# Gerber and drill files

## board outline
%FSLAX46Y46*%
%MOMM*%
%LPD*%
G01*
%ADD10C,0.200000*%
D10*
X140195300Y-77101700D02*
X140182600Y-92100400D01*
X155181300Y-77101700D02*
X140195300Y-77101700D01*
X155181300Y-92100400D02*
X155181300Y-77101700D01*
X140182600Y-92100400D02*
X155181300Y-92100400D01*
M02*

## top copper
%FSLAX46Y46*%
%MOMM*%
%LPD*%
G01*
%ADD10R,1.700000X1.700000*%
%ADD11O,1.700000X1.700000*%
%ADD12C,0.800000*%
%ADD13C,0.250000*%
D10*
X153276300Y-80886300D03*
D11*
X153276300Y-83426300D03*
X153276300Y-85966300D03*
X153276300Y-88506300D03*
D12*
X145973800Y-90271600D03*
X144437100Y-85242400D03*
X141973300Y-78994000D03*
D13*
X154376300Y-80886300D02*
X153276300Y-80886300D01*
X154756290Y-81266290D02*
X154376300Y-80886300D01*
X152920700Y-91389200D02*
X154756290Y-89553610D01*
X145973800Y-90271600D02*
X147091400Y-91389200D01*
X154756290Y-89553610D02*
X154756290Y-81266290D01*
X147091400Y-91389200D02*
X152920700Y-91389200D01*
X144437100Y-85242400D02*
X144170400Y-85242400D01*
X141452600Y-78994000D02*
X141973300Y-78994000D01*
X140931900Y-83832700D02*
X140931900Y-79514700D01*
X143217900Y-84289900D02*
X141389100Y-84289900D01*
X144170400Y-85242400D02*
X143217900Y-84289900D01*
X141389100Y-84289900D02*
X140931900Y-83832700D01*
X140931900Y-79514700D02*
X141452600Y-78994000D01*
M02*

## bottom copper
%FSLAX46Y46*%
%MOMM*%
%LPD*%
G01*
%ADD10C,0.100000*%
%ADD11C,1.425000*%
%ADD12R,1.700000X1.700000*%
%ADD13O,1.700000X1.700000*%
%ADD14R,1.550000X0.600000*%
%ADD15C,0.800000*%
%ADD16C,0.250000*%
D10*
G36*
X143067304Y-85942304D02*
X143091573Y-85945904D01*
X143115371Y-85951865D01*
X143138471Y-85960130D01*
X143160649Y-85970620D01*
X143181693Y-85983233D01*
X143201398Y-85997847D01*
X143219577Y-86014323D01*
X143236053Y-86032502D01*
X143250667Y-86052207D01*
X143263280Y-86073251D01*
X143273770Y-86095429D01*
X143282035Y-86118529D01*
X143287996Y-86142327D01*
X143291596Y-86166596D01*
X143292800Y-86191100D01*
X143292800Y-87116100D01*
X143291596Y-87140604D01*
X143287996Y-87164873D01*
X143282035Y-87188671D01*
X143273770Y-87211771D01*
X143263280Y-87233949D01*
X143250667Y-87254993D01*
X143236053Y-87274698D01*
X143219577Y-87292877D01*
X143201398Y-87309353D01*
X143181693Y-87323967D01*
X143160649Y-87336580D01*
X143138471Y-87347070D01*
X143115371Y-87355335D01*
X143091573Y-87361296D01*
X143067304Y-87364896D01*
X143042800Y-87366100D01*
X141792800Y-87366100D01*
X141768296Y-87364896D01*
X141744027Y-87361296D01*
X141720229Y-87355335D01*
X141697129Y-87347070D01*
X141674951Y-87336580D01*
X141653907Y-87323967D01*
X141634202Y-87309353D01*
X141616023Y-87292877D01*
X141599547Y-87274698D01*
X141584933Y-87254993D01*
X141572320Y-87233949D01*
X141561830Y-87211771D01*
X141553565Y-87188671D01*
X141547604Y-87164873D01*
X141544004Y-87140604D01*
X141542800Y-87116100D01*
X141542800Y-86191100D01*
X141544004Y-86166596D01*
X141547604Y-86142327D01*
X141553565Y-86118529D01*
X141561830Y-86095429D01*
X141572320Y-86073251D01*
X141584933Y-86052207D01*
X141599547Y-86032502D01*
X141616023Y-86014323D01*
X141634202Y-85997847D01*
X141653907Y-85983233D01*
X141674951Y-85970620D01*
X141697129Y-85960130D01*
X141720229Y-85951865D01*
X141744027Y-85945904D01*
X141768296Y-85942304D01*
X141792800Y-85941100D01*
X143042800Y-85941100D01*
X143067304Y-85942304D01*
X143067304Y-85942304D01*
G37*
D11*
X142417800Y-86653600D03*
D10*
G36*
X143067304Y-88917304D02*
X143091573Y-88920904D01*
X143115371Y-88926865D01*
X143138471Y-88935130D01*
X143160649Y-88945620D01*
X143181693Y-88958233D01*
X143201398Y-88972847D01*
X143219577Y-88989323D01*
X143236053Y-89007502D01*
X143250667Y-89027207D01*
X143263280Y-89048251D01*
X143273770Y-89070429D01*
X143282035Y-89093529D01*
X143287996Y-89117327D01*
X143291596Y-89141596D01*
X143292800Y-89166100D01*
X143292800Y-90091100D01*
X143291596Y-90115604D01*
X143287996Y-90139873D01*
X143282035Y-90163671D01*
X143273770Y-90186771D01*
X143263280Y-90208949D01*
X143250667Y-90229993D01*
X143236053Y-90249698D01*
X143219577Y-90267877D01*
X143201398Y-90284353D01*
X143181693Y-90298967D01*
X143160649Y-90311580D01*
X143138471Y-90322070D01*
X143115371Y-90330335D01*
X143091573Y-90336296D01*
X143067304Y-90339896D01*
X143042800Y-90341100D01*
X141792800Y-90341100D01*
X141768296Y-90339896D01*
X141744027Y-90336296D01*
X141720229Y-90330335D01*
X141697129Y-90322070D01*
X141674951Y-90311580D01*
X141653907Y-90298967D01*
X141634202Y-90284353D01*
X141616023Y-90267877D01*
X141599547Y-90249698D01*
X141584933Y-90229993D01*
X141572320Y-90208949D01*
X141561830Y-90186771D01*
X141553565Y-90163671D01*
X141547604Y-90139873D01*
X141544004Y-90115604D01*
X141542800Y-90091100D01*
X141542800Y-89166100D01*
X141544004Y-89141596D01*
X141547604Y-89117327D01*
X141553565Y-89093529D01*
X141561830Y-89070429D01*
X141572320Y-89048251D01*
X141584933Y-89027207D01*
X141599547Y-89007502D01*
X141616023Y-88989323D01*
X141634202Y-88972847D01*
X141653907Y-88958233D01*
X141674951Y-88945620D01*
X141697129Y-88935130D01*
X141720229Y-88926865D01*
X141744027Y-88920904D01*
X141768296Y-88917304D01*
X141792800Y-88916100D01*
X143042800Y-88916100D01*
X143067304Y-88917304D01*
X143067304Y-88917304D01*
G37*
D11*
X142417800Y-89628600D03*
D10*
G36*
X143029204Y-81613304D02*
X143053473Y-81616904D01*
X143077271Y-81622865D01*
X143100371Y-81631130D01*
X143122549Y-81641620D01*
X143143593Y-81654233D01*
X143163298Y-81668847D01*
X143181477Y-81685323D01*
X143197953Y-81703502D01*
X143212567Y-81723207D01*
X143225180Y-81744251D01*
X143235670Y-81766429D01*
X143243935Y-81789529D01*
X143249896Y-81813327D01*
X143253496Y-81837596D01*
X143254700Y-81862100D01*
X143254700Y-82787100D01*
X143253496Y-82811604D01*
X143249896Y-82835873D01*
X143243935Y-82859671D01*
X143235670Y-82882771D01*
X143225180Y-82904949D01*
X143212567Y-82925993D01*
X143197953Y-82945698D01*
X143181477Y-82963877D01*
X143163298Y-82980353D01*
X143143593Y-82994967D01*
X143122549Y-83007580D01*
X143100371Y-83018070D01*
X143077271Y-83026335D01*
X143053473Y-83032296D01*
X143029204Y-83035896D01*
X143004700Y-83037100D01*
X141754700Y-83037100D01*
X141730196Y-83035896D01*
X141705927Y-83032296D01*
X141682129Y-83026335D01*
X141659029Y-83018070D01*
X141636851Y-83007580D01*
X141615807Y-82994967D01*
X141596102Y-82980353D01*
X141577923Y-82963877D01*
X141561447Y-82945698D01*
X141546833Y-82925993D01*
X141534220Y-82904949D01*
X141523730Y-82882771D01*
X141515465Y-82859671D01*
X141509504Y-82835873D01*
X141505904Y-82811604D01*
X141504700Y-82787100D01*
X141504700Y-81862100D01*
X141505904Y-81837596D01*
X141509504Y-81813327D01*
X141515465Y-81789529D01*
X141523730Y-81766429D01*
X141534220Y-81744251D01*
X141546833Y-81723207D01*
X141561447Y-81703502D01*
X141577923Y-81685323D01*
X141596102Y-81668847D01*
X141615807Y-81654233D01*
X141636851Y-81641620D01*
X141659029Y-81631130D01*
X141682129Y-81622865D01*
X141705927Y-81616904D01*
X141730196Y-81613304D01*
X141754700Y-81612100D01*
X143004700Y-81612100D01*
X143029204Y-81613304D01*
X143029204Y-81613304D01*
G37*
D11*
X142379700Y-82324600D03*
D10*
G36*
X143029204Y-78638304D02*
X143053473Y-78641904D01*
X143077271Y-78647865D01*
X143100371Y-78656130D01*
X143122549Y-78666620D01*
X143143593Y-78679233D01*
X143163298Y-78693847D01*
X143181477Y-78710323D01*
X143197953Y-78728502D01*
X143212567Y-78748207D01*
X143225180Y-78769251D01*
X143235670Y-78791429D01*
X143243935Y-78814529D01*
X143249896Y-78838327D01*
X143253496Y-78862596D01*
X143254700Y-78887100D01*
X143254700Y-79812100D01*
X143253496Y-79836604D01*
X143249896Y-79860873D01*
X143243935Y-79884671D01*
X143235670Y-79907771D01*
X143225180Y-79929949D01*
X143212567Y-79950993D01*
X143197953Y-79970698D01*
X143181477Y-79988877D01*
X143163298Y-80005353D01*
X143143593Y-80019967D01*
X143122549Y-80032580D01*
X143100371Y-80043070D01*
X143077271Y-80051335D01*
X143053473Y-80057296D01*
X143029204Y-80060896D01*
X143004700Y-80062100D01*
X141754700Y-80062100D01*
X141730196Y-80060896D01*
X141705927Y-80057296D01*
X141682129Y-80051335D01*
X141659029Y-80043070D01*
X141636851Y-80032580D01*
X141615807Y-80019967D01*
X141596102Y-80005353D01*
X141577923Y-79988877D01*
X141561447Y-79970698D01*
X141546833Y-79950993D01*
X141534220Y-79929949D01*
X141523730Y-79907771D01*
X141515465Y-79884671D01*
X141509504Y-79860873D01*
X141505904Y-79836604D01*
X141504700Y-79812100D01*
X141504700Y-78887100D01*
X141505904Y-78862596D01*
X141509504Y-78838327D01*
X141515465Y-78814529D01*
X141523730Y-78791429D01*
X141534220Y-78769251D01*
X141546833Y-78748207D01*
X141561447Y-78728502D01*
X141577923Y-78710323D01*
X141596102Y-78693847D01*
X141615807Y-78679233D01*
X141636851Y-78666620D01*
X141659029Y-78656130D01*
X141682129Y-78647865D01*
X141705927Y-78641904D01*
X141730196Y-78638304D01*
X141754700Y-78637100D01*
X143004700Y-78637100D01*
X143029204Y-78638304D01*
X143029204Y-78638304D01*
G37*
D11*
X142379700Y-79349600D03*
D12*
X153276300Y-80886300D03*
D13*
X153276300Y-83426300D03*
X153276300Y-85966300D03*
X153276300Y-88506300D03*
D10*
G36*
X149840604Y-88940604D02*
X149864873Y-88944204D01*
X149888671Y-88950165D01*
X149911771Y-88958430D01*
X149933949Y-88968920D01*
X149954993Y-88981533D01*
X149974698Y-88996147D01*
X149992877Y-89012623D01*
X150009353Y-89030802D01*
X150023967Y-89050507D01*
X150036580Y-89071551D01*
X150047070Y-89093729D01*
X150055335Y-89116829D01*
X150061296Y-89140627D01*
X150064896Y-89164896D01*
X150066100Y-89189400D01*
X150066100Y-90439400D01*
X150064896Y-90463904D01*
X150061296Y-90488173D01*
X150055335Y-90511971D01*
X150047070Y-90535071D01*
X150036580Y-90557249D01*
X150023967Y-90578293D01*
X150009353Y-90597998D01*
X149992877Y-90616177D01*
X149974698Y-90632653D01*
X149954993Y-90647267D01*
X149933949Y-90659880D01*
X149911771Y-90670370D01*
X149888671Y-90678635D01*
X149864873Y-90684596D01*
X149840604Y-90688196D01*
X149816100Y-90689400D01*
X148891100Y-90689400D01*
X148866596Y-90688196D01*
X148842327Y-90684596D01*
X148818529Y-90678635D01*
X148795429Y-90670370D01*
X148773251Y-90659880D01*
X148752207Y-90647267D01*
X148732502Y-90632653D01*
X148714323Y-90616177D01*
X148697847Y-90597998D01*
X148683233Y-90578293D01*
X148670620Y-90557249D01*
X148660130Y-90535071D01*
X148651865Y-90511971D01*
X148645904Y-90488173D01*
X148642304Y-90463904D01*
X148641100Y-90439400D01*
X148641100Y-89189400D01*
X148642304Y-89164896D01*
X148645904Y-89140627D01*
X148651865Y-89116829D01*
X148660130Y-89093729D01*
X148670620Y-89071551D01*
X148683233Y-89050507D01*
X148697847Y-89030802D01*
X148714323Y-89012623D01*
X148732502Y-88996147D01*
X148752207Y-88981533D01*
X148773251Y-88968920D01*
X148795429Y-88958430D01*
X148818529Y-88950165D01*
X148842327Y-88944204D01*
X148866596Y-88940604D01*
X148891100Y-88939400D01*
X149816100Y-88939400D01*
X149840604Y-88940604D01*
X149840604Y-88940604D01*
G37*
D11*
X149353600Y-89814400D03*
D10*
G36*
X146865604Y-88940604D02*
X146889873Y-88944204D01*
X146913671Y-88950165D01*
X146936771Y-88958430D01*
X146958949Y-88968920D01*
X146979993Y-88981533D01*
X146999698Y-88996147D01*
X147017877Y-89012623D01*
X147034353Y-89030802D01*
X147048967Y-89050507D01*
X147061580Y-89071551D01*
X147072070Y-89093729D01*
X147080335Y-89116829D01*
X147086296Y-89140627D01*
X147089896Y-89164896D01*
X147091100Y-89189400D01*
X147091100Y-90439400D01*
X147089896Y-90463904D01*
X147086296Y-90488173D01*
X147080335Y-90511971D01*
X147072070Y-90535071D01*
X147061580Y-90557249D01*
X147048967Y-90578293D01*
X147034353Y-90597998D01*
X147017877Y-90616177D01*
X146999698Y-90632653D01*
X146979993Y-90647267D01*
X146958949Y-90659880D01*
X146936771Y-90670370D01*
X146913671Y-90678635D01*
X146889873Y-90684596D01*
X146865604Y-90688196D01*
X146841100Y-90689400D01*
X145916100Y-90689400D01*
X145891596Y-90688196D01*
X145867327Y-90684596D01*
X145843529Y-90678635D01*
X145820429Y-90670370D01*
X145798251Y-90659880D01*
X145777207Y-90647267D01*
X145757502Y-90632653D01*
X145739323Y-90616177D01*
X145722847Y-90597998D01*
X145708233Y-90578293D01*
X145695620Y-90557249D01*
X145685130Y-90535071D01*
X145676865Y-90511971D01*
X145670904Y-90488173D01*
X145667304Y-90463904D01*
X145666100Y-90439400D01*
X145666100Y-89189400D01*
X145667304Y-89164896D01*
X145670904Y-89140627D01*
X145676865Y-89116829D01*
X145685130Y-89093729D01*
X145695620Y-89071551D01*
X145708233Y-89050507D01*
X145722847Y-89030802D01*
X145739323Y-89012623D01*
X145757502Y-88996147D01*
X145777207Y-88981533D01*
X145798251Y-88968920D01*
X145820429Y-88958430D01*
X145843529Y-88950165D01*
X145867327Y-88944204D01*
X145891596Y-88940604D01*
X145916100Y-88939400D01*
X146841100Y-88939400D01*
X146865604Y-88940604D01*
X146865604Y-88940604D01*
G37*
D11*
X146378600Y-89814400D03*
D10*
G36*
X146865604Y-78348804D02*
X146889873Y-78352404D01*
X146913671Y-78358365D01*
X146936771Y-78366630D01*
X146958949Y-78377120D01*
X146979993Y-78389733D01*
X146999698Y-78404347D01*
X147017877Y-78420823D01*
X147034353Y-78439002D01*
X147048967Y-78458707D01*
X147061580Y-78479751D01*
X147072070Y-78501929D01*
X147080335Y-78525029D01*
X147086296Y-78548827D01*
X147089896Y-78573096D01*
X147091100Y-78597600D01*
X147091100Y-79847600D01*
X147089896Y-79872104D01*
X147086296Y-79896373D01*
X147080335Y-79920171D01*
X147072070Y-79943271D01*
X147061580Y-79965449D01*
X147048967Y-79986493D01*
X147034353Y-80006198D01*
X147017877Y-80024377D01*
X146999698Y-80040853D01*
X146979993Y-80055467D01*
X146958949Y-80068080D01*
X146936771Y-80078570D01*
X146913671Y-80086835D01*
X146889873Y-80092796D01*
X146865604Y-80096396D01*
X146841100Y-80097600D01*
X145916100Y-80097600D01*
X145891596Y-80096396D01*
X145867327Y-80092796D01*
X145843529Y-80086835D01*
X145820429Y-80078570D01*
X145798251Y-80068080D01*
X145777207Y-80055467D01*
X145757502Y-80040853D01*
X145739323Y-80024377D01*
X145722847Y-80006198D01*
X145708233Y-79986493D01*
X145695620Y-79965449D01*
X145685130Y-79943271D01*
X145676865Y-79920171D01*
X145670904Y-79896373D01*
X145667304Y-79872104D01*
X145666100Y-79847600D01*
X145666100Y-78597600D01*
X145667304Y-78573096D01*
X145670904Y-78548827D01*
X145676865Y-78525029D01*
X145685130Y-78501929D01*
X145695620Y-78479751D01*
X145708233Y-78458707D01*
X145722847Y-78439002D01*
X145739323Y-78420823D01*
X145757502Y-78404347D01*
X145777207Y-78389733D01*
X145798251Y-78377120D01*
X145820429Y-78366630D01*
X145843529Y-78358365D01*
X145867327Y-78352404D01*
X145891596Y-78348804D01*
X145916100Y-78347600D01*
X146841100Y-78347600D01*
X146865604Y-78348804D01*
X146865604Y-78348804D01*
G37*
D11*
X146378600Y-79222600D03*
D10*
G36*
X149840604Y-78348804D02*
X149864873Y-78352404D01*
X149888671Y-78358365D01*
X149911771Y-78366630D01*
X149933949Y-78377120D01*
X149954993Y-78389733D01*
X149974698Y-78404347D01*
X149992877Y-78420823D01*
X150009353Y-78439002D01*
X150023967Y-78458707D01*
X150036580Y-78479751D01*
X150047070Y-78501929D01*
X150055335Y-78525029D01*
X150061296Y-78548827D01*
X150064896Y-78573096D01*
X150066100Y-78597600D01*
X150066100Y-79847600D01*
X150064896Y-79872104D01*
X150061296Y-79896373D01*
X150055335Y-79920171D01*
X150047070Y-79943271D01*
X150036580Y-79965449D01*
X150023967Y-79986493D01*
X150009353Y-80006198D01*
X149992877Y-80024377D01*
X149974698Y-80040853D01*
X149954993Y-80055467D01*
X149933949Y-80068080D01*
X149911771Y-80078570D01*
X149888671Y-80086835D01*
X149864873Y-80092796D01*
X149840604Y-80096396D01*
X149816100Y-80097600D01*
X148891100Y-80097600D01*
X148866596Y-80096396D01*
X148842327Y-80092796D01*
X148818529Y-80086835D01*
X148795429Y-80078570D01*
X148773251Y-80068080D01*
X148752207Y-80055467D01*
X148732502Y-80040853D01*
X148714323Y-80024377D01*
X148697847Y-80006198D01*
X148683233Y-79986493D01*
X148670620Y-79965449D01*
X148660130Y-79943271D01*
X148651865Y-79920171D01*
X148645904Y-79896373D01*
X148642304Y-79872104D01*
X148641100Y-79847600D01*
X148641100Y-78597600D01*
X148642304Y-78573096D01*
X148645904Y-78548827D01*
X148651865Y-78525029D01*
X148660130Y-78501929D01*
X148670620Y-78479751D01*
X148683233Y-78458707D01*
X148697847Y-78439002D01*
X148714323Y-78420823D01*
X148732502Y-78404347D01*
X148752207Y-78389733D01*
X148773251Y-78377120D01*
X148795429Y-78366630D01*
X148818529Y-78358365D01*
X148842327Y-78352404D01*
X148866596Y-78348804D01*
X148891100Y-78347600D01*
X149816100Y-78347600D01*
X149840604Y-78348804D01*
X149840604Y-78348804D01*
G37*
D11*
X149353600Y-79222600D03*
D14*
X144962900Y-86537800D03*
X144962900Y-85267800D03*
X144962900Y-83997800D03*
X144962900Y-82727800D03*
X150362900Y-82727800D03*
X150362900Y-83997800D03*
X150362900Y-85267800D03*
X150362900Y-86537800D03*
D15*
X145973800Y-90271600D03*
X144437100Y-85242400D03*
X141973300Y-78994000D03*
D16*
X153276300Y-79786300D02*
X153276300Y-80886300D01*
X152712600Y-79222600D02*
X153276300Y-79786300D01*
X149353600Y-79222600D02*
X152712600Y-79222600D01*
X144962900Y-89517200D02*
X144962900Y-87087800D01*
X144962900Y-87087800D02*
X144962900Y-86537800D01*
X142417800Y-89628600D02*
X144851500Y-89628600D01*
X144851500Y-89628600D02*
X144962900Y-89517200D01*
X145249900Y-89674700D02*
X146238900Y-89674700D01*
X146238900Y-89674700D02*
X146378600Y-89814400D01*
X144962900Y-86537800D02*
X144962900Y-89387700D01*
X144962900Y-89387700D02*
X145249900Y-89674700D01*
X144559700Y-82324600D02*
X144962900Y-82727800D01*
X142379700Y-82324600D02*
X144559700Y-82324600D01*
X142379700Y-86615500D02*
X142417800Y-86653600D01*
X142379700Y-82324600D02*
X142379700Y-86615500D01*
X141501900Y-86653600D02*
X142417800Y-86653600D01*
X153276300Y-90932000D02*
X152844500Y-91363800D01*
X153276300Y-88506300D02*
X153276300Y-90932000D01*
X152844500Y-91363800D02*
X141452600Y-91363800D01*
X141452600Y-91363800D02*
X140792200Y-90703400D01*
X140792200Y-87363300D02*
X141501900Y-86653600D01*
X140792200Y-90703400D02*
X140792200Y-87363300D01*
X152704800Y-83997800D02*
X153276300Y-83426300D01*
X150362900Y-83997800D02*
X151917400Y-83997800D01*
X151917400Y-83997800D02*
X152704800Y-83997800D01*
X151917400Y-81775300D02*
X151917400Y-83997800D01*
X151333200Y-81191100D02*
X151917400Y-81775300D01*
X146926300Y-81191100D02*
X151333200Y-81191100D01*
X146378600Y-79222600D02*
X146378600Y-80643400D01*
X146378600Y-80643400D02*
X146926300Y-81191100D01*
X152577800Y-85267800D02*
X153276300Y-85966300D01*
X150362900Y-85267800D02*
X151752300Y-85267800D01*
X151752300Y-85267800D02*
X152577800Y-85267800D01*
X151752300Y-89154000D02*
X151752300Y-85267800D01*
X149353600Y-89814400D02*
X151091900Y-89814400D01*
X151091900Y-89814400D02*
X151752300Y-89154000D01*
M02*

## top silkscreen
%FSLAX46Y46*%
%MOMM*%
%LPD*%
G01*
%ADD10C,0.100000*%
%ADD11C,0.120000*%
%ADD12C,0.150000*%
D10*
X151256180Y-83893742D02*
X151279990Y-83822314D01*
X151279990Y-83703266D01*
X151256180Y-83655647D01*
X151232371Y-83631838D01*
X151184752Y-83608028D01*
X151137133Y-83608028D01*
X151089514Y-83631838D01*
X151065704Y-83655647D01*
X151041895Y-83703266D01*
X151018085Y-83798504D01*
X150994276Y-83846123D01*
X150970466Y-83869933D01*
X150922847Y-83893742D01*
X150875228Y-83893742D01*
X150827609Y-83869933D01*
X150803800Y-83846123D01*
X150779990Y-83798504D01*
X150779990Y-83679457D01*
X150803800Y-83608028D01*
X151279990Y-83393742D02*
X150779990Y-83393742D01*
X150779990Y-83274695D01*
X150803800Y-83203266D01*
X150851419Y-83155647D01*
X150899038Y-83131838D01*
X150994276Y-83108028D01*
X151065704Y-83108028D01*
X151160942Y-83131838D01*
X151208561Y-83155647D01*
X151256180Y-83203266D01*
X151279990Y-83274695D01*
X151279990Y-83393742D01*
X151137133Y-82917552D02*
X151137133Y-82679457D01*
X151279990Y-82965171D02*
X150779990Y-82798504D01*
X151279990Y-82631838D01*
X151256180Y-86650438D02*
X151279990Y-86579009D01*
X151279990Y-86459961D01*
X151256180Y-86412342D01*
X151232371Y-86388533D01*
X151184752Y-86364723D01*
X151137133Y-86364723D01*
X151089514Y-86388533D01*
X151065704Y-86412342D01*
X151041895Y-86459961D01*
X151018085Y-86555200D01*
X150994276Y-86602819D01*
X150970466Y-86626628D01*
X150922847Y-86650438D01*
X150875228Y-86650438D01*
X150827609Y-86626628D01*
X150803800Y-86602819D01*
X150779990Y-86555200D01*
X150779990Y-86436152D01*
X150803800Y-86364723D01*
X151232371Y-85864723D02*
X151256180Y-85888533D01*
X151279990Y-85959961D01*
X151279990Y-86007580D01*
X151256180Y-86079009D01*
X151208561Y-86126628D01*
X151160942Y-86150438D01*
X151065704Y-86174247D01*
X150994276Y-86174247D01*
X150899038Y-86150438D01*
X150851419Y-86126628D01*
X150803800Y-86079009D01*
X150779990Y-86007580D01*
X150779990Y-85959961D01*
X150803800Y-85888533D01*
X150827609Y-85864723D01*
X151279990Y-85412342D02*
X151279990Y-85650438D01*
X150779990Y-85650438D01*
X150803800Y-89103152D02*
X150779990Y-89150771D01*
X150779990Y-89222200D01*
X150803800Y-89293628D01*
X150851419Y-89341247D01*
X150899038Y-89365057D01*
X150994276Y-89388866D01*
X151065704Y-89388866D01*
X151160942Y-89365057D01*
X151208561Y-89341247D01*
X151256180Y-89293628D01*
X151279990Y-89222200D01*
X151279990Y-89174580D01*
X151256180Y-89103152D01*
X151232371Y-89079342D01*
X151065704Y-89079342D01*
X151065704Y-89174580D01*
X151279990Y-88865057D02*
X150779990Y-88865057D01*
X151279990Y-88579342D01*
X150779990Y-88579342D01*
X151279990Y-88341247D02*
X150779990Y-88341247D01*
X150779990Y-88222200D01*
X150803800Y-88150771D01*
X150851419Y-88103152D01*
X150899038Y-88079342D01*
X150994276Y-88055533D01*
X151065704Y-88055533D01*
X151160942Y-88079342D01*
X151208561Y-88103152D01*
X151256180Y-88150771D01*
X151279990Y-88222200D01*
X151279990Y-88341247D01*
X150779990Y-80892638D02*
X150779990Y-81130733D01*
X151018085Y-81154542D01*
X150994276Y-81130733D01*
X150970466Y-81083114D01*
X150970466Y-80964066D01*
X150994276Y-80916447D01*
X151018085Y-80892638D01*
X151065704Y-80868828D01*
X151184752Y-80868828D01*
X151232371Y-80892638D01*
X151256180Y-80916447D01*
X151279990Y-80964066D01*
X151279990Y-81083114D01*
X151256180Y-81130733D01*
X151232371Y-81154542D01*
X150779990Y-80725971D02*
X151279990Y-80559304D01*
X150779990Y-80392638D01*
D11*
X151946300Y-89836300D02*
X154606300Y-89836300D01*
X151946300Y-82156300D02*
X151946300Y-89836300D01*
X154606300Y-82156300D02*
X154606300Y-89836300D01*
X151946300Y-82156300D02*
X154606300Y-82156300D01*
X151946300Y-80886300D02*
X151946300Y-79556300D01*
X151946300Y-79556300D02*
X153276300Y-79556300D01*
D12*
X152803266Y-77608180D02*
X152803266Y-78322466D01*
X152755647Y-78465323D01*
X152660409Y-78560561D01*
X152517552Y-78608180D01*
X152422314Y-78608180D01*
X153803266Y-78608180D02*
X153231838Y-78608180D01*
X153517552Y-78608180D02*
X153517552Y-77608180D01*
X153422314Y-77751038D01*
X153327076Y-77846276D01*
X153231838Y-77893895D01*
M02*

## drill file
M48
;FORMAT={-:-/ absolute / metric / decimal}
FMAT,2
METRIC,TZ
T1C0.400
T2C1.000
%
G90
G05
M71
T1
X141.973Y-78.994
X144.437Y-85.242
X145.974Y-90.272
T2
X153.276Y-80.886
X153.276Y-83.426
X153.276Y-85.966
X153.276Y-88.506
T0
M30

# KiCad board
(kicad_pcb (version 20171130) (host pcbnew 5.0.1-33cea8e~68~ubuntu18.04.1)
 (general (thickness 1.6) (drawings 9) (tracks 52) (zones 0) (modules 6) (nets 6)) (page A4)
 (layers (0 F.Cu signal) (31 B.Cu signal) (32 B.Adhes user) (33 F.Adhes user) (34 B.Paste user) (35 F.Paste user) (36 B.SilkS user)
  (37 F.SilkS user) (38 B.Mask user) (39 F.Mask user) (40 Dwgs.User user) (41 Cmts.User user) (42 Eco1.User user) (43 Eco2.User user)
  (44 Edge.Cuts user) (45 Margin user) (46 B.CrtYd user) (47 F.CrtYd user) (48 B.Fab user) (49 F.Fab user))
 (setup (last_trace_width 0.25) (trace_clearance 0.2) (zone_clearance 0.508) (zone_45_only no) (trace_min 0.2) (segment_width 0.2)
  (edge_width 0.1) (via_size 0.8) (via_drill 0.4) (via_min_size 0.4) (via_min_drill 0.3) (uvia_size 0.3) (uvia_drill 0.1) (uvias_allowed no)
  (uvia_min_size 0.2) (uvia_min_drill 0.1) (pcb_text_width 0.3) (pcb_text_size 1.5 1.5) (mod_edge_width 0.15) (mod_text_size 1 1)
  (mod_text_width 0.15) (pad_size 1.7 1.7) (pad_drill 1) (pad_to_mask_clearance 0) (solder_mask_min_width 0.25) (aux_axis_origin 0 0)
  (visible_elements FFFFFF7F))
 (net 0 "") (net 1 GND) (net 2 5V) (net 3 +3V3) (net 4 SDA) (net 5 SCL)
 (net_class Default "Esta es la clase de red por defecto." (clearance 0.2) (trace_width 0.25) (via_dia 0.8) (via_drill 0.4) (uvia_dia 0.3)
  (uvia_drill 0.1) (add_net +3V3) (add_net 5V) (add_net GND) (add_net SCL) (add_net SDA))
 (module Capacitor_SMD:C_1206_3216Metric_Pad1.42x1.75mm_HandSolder (layer B.Cu) (at 142.4178 88.1411 90)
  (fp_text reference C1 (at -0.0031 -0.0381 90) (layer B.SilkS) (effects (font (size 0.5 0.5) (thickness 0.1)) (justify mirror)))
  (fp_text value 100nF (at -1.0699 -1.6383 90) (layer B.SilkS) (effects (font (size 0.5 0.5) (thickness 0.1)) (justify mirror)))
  (pad 2 smd roundrect (at 1.4875 0 90) (size 1.425 1.75) (layers B.Cu B.Paste B.Mask) (roundrect_rratio 0.175439) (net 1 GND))
  (pad 1 smd roundrect (at -1.4875 0 90) (size 1.425 1.75) (layers B.Cu B.Paste B.Mask) (roundrect_rratio 0.175439) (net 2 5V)))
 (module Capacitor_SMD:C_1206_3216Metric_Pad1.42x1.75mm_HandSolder (layer B.Cu) (at 142.3797 80.8371 270)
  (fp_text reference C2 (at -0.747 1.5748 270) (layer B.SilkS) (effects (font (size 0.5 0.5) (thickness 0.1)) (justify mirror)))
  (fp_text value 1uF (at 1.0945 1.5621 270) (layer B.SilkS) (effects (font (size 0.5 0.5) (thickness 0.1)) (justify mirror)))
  (pad 2 smd roundrect (at 1.4875 0 270) (size 1.425 1.75) (layers B.Cu B.Paste B.Mask) (roundrect_rratio 0.175439) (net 1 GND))
  (pad 1 smd roundrect (at -1.4875 0 270) (size 1.425 1.75) (layers B.Cu B.Paste B.Mask) (roundrect_rratio 0.175439) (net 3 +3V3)))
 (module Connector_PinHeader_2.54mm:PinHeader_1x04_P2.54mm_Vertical (layer F.Cu) (at 153.2763 80.8863)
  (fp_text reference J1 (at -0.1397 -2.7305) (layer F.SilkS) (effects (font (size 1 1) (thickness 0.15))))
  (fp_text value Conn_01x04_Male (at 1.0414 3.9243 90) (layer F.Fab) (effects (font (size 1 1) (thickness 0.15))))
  (fp_line (start -1.33 8.95) (end 1.33 8.95) (layer F.SilkS) (width 0.12))
  (fp_line (start -1.33 1.27) (end -1.33 8.95) (layer F.SilkS) (width 0.12))
  (fp_line (start 1.33 1.27) (end 1.33 8.95) (layer F.SilkS) (width 0.12))
  (fp_line (start -1.33 1.27) (end 1.33 1.27) (layer F.SilkS) (width 0.12))
  (fp_line (start -1.33 0) (end -1.33 -1.33) (layer F.SilkS) (width 0.12))
  (fp_line (start -1.33 -1.33) (end 0 -1.33) (layer F.SilkS) (width 0.12))
  (pad 1 thru_hole rect (at 0 0) (size 1.7 1.7) (drill 1) (layers *.Cu *.Mask) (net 2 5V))
  (pad 2 thru_hole oval (at 0 2.54) (size 1.7 1.7) (drill 1) (layers *.Cu *.Mask) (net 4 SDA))
  (pad 3 thru_hole oval (at 0 5.08) (size 1.7 1.7) (drill 1) (layers *.Cu *.Mask) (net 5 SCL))
  (pad 4 thru_hole oval (at 0 7.62) (size 1.7 1.7) (drill 1) (layers *.Cu *.Mask) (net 1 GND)))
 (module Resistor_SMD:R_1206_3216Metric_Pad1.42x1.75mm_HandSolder (layer B.Cu) (at 147.8661 89.8144)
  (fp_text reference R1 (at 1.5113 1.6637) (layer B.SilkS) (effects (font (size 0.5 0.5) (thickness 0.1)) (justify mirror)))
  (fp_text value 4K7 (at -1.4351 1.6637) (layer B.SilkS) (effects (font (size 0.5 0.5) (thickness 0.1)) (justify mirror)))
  (pad 2 smd roundrect (at 1.4875 0) (size 1.425 1.75) (layers B.Cu B.Paste B.Mask) (roundrect_rratio 0.175439) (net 5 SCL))
  (pad 1 smd roundrect (at -1.4875 0) (size 1.425 1.75) (layers B.Cu B.Paste B.Mask) (roundrect_rratio 0.175439) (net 2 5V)))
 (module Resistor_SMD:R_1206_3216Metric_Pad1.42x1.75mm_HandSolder (layer B.Cu) (at 147.8661 79.2226 180)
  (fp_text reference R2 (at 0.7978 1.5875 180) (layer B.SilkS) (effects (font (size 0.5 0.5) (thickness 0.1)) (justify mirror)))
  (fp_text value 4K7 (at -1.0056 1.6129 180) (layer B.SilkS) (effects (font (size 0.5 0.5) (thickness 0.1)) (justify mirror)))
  (pad 2 smd roundrect (at 1.4875 0 180) (size 1.425 1.75) (layers B.Cu B.Paste B.Mask) (roundrect_rratio 0.175439) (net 4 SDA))
  (pad 1 smd roundrect (at -1.4875 0 180) (size 1.425 1.75) (layers B.Cu B.Paste B.Mask) (roundrect_rratio 0.175439) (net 2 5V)))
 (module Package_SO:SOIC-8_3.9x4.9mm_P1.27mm (layer B.Cu) (at 147.6629 84.6328)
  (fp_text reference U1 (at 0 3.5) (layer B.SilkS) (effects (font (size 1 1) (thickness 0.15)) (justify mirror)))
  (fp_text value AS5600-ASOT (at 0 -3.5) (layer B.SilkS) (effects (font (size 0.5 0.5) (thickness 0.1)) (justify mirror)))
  (pad 1 smd rect (at -2.7 1.905) (size 1.55 0.6) (layers B.Cu B.Paste B.Mask) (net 2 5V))
  (pad 2 smd rect (at -2.7 0.635) (size 1.55 0.6) (layers B.Cu B.Paste B.Mask) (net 3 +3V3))
  (pad 3 smd rect (at -2.7 -0.635) (size 1.55 0.6) (layers B.Cu B.Paste B.Mask))
  (pad 4 smd rect (at -2.7 -1.905) (size 1.55 0.6) (layers B.Cu B.Paste B.Mask) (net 1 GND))
  (pad 5 smd rect (at 2.7 -1.905) (size 1.55 0.6) (layers B.Cu B.Paste B.Mask))
  (pad 6 smd rect (at 2.7 -0.635) (size 1.55 0.6) (layers B.Cu B.Paste B.Mask) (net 4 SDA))
  (pad 7 smd rect (at 2.7 0.635) (size 1.55 0.6) (layers B.Cu B.Paste B.Mask) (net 5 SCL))
  (pad 8 smd rect (at 2.7 1.905) (size 1.55 0.6) (layers B.Cu B.Paste B.Mask)))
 (gr_line (start 140.1953 77.1017) (end 140.1826 92.1004) (layer Edge.Cuts) (width 0.2))
 (gr_line (start 155.1813 77.1017) (end 140.1953 77.1017) (layer Edge.Cuts) (width 0.2))
 (gr_line (start 155.1813 92.1004) (end 155.1813 77.1017) (layer Edge.Cuts) (width 0.2))
 (gr_line (start 140.1826 92.1004) (end 155.1813 92.1004) (layer Edge.Cuts) (width 0.2))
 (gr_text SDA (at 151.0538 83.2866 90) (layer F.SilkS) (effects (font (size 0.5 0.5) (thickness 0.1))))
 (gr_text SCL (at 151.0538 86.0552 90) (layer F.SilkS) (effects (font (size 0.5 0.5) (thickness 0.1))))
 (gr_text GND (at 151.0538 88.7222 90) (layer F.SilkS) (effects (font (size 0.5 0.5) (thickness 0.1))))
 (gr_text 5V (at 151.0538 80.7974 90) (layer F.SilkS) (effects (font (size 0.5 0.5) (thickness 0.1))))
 (via (at 145.9738 90.2716) (size 0.8) (drill 0.4) (layers F.Cu B.Cu) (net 2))
 (segment (start 153.2763 79.7863) (end 153.2763 80.8863) (width 0.25) (layer B.Cu) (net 2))
 (segment (start 152.7126 79.2226) (end 153.2763 79.7863) (width 0.25) (layer B.Cu) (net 2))
 (segment (start 149.3536 79.2226) (end 152.7126 79.2226) (width 0.25) (layer B.Cu) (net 2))
 (segment (start 154.3763 80.8863) (end 153.2763 80.8863) (width 0.25) (layer F.Cu) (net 2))
 (segment (start 154.75629 81.26629) (end 154.3763 80.8863) (width 0.25) (layer F.Cu) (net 2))
 (segment (start 152.9207 91.3892) (end 154.75629 89.55361) (width 0.25) (layer F.Cu) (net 2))
 (segment (start 145.9738 90.2716) (end 147.0914 91.3892) (width 0.25) (layer F.Cu) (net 2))
 (segment (start 154.75629 89.55361) (end 154.75629 81.26629) (width 0.25) (layer F.Cu) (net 2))
 (segment (start 147.0914 91.3892) (end 152.9207 91.3892) (width 0.25) (layer F.Cu) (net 2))
 (segment (start 144.9629 89.5172) (end 144.9629 87.0878) (width 0.25) (layer B.Cu) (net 2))
 (segment (start 144.9629 87.0878) (end 144.9629 86.5378) (width 0.25) (layer B.Cu) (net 2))
 (segment (start 142.4178 89.6286) (end 144.8515 89.6286) (width 0.25) (layer B.Cu) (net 2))
 (segment (start 144.8515 89.6286) (end 144.9629 89.5172) (width 0.25) (layer B.Cu) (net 2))
 (segment (start 145.2499 89.6747) (end 146.2389 89.6747) (width 0.25) (layer B.Cu) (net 2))
 (segment (start 146.2389 89.6747) (end 146.3786 89.8144) (width 0.25) (layer B.Cu) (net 2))
 (segment (start 144.9629 86.5378) (end 144.9629 89.3877) (width 0.25) (layer B.Cu) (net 2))
 (segment (start 144.9629 89.3877) (end 145.2499 89.6747) (width 0.25) (layer B.Cu) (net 2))
 (segment (start 144.5597 82.3246) (end 144.9629 82.7278) (width 0.25) (layer B.Cu) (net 1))
 (segment (start 142.3797 82.3246) (end 144.5597 82.3246) (width 0.25) (layer B.Cu) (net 1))
 (segment (start 142.3797 86.6155) (end 142.4178 86.6536) (width 0.25) (layer B.Cu) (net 1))
 (segment (start 142.3797 82.3246) (end 142.3797 86.6155) (width 0.25) (layer B.Cu) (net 1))
 (segment (start 141.5019 86.6536) (end 142.4178 86.6536) (width 0.25) (layer B.Cu) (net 1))
 (segment (start 153.2763 90.932) (end 152.8445 91.3638) (width 0.25) (layer B.Cu) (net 1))
 (segment (start 153.2763 88.5063) (end 153.2763 90.932) (width 0.25) (layer B.Cu) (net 1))
 (segment (start 152.8445 91.3638) (end 141.4526 91.3638) (width 0.25) (layer B.Cu) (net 1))
 (segment (start 141.4526 91.3638) (end 140.7922 90.7034) (width 0.25) (layer B.Cu) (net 1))
 (segment (start 140.7922 87.3633) (end 141.5019 86.6536) (width 0.25) (layer B.Cu) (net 1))
 (segment (start 140.7922 90.7034) (end 140.7922 87.3633) (width 0.25) (layer B.Cu) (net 1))
 (via (at 144.4371 85.2424) (size 0.8) (drill 0.4) (layers F.Cu B.Cu) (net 3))
 (via (at 141.9733 78.994) (size 0.8) (drill 0.4) (layers F.Cu B.Cu) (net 3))
 (segment (start 144.4371 85.2424) (end 144.1704 85.2424) (width 0.25) (layer F.Cu) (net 3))
 (segment (start 141.4526 78.994) (end 141.9733 78.994) (width 0.25) (layer F.Cu) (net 3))
 (segment (start 140.9319 83.8327) (end 140.9319 79.5147) (width 0.25) (layer F.Cu) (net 3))
 (segment (start 143.2179 84.2899) (end 141.3891 84.2899) (width 0.25) (layer F.Cu) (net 3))
 (segment (start 144.1704 85.2424) (end 143.2179 84.2899) (width 0.25) (layer F.Cu) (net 3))
 (segment (start 141.3891 84.2899) (end 140.9319 83.8327) (width 0.25) (layer F.Cu) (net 3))
 (segment (start 140.9319 79.5147) (end 141.4526 78.994) (width 0.25) (layer F.Cu) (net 3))
 (segment (start 152.7048 83.9978) (end 153.2763 83.4263) (width 0.25) (layer B.Cu) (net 4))
 (segment (start 150.3629 83.9978) (end 151.9174 83.9978) (width 0.25) (layer B.Cu) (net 4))
 (segment (start 151.9174 83.9978) (end 152.7048 83.9978) (width 0.25) (layer B.Cu) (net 4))
 (segment (start 151.9174 81.7753) (end 151.9174 83.9978) (width 0.25) (layer B.Cu) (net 4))
 (segment (start 151.3332 81.1911) (end 151.9174 81.7753) (width 0.25) (layer B.Cu) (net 4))
 (segment (start 146.9263 81.1911) (end 151.3332 81.1911) (width 0.25) (layer B.Cu) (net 4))
 (segment (start 146.3786 79.2226) (end 146.3786 80.6434) (width 0.25) (layer B.Cu) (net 4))
 (segment (start 146.3786 80.6434) (end 146.9263 81.1911) (width 0.25) (layer B.Cu) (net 4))
 (segment (start 152.5778 85.2678) (end 153.2763 85.9663) (width 0.25) (layer B.Cu) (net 5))
 (segment (start 150.3629 85.2678) (end 151.7523 85.2678) (width 0.25) (layer B.Cu) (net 5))
 (segment (start 151.7523 85.2678) (end 152.5778 85.2678) (width 0.25) (layer B.Cu) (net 5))
 (segment (start 151.7523 89.154) (end 151.7523 85.2678) (width 0.25) (layer B.Cu) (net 5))
 (segment (start 149.3536 89.8144) (end 151.0919 89.8144) (width 0.25) (layer B.Cu) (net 5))
 (segment (start 151.0919 89.8144) (end 151.7523 89.154) (width 0.25) (layer B.Cu) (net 5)))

